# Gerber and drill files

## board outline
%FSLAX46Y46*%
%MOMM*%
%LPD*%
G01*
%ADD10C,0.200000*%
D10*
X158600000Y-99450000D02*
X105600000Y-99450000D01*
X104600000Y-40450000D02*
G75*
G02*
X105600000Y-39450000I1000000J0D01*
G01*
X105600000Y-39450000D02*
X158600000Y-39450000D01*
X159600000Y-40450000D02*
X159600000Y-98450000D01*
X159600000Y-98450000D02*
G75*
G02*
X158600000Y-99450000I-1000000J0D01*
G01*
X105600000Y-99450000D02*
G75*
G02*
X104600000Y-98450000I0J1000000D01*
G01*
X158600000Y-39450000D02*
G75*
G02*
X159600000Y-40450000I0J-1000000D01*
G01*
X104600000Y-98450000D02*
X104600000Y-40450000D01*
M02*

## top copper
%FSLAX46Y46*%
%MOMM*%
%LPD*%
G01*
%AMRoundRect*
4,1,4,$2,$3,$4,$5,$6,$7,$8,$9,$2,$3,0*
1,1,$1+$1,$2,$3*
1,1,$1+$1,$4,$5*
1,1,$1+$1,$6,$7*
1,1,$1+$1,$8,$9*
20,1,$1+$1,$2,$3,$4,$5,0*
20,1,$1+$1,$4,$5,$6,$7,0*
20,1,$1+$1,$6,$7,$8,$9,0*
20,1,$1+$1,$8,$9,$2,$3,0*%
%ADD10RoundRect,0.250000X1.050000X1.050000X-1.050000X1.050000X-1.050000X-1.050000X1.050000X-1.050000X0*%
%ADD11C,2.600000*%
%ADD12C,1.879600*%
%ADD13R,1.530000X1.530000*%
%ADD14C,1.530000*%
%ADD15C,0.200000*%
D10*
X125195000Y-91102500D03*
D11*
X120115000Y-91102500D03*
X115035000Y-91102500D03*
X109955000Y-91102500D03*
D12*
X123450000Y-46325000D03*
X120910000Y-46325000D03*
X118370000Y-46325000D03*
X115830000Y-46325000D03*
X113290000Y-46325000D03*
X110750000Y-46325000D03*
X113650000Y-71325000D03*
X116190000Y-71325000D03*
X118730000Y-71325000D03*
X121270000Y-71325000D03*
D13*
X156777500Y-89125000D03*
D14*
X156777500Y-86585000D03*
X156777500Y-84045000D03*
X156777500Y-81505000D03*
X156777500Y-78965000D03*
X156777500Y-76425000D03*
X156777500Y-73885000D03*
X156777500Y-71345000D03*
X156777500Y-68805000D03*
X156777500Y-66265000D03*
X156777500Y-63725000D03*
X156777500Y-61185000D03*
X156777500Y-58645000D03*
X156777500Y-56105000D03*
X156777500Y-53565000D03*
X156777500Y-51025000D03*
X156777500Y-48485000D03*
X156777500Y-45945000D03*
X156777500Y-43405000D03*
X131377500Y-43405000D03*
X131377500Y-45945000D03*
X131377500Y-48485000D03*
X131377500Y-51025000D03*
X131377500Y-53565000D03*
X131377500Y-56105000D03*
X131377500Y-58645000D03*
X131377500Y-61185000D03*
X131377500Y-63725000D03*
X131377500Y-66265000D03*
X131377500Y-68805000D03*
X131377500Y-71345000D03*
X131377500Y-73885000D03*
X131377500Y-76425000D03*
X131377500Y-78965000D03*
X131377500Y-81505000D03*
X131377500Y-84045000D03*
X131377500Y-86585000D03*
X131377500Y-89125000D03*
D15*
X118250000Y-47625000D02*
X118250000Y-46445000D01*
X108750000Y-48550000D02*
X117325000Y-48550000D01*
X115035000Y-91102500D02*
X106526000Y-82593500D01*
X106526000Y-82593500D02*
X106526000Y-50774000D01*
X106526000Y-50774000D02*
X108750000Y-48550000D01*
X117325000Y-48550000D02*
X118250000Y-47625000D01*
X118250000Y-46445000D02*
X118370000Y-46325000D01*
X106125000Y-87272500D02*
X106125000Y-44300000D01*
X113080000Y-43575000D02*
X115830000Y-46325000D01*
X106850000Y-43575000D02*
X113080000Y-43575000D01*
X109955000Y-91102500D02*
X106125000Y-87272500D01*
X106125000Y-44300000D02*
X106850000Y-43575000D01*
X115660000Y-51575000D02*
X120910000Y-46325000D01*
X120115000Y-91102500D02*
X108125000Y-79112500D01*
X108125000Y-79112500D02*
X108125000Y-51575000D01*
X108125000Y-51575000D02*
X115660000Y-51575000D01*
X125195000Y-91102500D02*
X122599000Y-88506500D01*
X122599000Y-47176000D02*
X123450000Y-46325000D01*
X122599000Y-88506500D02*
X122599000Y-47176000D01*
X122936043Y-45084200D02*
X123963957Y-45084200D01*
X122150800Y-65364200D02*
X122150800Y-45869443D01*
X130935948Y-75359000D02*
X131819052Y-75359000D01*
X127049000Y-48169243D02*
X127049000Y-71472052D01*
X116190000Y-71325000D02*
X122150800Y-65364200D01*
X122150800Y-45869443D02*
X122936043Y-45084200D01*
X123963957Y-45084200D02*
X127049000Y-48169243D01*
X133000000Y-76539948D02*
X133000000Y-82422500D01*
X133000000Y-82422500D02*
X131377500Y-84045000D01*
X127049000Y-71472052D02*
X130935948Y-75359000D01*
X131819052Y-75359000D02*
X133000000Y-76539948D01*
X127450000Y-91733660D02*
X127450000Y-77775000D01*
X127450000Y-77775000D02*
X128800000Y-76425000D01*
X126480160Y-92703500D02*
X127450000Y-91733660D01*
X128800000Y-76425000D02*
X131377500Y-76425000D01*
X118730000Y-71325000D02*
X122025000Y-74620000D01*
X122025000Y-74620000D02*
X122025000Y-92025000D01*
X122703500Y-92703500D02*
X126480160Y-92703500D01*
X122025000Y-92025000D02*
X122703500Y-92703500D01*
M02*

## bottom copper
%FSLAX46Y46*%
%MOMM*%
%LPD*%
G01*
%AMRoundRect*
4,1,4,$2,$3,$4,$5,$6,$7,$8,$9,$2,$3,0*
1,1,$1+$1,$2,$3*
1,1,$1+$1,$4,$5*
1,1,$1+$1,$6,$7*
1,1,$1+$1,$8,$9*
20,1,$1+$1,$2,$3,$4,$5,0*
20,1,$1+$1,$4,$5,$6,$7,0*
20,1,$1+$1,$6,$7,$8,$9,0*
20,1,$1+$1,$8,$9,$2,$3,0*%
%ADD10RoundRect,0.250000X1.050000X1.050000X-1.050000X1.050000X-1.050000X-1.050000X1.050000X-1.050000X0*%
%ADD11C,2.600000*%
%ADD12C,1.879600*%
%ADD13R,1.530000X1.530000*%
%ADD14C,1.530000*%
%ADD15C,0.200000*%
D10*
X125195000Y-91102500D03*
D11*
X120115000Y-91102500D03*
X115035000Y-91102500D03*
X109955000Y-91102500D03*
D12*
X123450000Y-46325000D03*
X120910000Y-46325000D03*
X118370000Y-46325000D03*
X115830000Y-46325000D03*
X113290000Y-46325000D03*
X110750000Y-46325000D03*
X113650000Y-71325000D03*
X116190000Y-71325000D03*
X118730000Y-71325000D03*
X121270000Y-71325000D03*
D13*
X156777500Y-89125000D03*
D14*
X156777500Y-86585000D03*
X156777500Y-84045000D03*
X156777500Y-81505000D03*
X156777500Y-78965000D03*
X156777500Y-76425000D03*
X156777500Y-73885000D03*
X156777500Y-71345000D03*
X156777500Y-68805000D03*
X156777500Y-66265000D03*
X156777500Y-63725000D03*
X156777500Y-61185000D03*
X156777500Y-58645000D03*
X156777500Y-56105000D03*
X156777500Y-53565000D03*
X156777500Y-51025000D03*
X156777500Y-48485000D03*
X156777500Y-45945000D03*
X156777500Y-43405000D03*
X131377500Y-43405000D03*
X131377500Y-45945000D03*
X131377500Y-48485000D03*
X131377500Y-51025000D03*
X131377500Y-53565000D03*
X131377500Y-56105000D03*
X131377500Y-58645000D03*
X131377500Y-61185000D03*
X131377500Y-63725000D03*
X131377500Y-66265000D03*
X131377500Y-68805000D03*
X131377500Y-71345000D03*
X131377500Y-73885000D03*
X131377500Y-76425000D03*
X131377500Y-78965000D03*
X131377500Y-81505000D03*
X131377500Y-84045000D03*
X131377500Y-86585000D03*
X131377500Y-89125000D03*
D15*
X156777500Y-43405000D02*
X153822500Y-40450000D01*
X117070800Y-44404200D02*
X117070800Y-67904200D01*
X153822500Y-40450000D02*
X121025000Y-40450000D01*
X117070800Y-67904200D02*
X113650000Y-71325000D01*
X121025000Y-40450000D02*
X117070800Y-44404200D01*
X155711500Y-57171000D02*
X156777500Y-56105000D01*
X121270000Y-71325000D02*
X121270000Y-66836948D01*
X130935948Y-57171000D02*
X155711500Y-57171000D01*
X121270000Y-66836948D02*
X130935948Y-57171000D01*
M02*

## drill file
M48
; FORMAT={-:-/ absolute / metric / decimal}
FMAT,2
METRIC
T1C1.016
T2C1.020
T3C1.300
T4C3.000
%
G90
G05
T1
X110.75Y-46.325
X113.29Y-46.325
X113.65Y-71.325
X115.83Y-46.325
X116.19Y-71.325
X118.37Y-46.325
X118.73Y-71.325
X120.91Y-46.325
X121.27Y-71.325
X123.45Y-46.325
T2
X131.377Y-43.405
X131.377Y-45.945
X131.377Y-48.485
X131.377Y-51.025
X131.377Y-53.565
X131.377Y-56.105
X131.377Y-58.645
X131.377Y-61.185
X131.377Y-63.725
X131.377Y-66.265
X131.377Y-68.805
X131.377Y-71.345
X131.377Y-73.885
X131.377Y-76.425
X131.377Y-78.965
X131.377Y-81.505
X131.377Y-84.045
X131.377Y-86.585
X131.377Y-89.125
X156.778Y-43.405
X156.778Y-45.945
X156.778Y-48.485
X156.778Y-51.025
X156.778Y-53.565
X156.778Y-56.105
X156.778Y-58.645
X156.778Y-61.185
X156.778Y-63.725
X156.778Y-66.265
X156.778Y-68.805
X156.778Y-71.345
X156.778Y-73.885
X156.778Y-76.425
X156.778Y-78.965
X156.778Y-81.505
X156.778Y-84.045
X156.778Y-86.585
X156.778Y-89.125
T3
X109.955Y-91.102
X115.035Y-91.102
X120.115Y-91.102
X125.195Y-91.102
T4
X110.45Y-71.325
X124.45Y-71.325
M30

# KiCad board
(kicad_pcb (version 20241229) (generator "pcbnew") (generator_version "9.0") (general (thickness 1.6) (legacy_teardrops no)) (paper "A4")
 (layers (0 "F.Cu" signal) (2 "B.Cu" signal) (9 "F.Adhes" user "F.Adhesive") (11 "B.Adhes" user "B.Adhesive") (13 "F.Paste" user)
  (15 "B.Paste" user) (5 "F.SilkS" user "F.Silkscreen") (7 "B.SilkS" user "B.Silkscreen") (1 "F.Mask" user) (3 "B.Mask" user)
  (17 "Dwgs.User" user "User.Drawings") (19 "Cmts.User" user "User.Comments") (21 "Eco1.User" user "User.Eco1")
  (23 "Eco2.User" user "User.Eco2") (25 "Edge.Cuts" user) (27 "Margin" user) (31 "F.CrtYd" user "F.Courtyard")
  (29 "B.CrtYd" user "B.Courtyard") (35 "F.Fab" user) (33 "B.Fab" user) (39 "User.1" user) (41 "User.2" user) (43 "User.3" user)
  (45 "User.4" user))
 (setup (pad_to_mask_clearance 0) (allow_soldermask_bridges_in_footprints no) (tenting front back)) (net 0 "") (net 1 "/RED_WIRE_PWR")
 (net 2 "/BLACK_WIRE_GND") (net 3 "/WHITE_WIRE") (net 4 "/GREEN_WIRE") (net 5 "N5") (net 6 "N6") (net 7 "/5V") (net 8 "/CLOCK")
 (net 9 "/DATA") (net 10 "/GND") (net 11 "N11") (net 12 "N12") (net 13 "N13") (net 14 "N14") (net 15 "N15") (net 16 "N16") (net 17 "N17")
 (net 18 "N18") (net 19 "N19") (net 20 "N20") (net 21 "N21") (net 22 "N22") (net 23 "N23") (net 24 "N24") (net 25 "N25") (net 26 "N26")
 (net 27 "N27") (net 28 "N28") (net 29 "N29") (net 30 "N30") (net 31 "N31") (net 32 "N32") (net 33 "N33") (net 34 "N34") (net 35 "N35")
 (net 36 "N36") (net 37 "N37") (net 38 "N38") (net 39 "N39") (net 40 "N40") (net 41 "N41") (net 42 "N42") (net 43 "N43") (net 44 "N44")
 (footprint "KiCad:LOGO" (layer "F.Cu") (at 138.975 67.075)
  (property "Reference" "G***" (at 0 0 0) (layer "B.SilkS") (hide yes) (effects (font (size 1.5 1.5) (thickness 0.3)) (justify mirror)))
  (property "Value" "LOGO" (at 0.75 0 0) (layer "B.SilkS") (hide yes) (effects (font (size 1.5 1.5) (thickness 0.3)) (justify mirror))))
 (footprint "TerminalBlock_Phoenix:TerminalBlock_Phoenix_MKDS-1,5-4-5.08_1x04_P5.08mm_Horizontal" (layer "F.Cu") (at 125.195 91.1025 180)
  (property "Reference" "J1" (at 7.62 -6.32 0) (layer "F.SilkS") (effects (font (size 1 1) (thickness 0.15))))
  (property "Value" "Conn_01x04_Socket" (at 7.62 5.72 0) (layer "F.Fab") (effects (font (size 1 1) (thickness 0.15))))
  (pad "1" thru_hole roundrect (at 0 0 180) (size 2.6 2.6) (drill 1.3) (layers "*.Cu" "*.Mask") (remove_unused_layers no)
   (roundrect_rratio 0.096154) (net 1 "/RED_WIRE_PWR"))
  (pad "2" thru_hole circle (at 5.08 0 180) (size 2.6 2.6) (drill 1.3) (layers "*.Cu" "*.Mask") (remove_unused_layers no)
   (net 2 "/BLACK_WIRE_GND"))
  (pad "3" thru_hole circle (at 10.16 0 180) (size 2.6 2.6) (drill 1.3) (layers "*.Cu" "*.Mask") (remove_unused_layers no)
   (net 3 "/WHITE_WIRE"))
  (pad "4" thru_hole circle (at 15.24 0 180) (size 2.6 2.6) (drill 1.3) (layers "*.Cu" "*.Mask") (remove_unused_layers no)
   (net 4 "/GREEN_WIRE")))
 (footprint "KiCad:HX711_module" (layer "F.Cu") (at 117.45 59.325 -90)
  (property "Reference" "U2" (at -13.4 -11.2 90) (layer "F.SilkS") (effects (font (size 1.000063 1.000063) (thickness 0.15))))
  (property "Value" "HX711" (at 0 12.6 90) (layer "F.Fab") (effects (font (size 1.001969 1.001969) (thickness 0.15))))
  (pad "" np_thru_hole circle (at 12 -7 270) (size 3 3) (drill 3) (layers "*.Cu" "*.Mask"))
  (pad "" np_thru_hole circle (at 12 7 270) (size 3 3) (drill 3) (layers "*.Cu" "*.Mask"))
  (pad "1" thru_hole circle (at -13 -6 270) (size 1.8796 1.8796) (drill 1.016) (layers "*.Cu" "*.Mask") (remove_unused_layers no)
   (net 1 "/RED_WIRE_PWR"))
  (pad "2" thru_hole circle (at -13 -3.46 270) (size 1.8796 1.8796) (drill 1.016) (layers "*.Cu" "*.Mask") (remove_unused_layers no)
   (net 2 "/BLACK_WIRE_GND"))
  (pad "3" thru_hole circle (at -13 -0.92 270) (size 1.8796 1.8796) (drill 1.016) (layers "*.Cu" "*.Mask") (remove_unused_layers no)
   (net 3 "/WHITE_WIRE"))
  (pad "4" thru_hole circle (at -13 1.62 270) (size 1.8796 1.8796) (drill 1.016) (layers "*.Cu" "*.Mask") (remove_unused_layers no)
   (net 4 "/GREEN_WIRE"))
  (pad "5" thru_hole circle (at -13 4.16 270) (size 1.8796 1.8796) (drill 1.016) (layers "*.Cu" "*.Mask") (remove_unused_layers no)
   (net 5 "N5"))
  (pad "6" thru_hole circle (at -13 6.7 270) (size 1.8796 1.8796) (drill 1.016) (layers "*.Cu" "*.Mask") (remove_unused_layers no)
   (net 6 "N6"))
  (pad "7" thru_hole circle (at 12 3.8 270) (size 1.8796 1.8796) (drill 1.016) (layers "*.Cu" "*.Mask") (remove_unused_layers no)
   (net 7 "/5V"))
  (pad "8" thru_hole circle (at 12 1.26 270) (size 1.8796 1.8796) (drill 1.016) (layers "*.Cu" "*.Mask") (remove_unused_layers no)
   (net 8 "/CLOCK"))
  (pad "9" thru_hole circle (at 12 -1.28 270) (size 1.8796 1.8796) (drill 1.016) (layers "*.Cu" "*.Mask") (remove_unused_layers no)
   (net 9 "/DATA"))
  (pad "10" thru_hole circle (at 12 -3.82 270) (size 1.8796 1.8796) (drill 1.016) (layers "*.Cu" "*.Mask") (remove_unused_layers no)
   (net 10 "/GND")))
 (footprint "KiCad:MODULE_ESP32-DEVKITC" (layer "F.Cu") (at 144.0775 66.275 180)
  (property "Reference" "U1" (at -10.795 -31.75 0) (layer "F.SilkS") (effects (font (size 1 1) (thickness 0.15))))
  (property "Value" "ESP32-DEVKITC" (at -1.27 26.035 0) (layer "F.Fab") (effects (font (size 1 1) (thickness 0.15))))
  (pad "1" thru_hole rect (at -12.7 -22.85 180) (size 1.53 1.53) (drill 1.02) (layers "*.Cu" "*.Mask") (remove_unused_layers no)
   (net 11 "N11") (solder_mask_margin 0.102))
  (pad "2" thru_hole circle (at -12.7 -20.31 180) (size 1.53 1.53) (drill 1.02) (layers "*.Cu" "*.Mask") (remove_unused_layers no)
   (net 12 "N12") (solder_mask_margin 0.102))
  (pad "3" thru_hole circle (at -12.7 -17.77 180) (size 1.53 1.53) (drill 1.02) (layers "*.Cu" "*.Mask") (remove_unused_layers no)
   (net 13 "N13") (solder_mask_margin 0.102))
  (pad "4" thru_hole circle (at -12.7 -15.23 180) (size 1.53 1.53) (drill 1.02) (layers "*.Cu" "*.Mask") (remove_unused_layers no)
   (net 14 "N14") (solder_mask_margin 0.102))
  (pad "5" thru_hole circle (at -12.7 -12.69 180) (size 1.53 1.53) (drill 1.02) (layers "*.Cu" "*.Mask") (remove_unused_layers no)
   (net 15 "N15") (solder_mask_margin 0.102))
  (pad "6" thru_hole circle (at -12.7 -10.15 180) (size 1.53 1.53) (drill 1.02) (layers "*.Cu" "*.Mask") (remove_unused_layers no)
   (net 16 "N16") (solder_mask_margin 0.102))
  (pad "7" thru_hole circle (at -12.7 -7.61 180) (size 1.53 1.53) (drill 1.02) (layers "*.Cu" "*.Mask") (remove_unused_layers no)
   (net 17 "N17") (solder_mask_margin 0.102))
  (pad "8" thru_hole circle (at -12.7 -5.07 180) (size 1.53 1.53) (drill 1.02) (layers "*.Cu" "*.Mask") (remove_unused_layers no)
   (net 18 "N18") (solder_mask_margin 0.102))
  (pad "9" thru_hole circle (at -12.7 -2.53 180) (size 1.53 1.53) (drill 1.02) (layers "*.Cu" "*.Mask") (remove_unused_layers no)
   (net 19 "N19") (solder_mask_margin 0.102))
  (pad "10" thru_hole circle (at -12.7 0.01 180) (size 1.53 1.53) (drill 1.02) (layers "*.Cu" "*.Mask") (remove_unused_layers no)
   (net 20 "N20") (solder_mask_margin 0.102))
  (pad "11" thru_hole circle (at -12.7 2.55 180) (size 1.53 1.53) (drill 1.02) (layers "*.Cu" "*.Mask") (remove_unused_layers no)
   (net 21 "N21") (solder_mask_margin 0.102))
  (pad "12" thru_hole circle (at -12.7 5.09 180) (size 1.53 1.53) (drill 1.02) (layers "*.Cu" "*.Mask") (remove_unused_layers no)
   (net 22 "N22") (solder_mask_margin 0.102))
  (pad "13" thru_hole circle (at -12.7 7.63 180) (size 1.53 1.53) (drill 1.02) (layers "*.Cu" "*.Mask") (remove_unused_layers no)
   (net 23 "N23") (solder_mask_margin 0.102))
  (pad "14" thru_hole circle (at -12.7 10.17 180) (size 1.53 1.53) (drill 1.02) (layers "*.Cu" "*.Mask") (remove_unused_layers no)
   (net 10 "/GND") (solder_mask_margin 0.102))
  (pad "15" thru_hole circle (at -12.7 12.71 180) (size 1.53 1.53) (drill 1.02) (layers "*.Cu" "*.Mask") (remove_unused_layers no)
   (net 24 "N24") (solder_mask_margin 0.102))
  (pad "16" thru_hole circle (at -12.7 15.25 180) (size 1.53 1.53) (drill 1.02) (layers "*.Cu" "*.Mask") (remove_unused_layers no)
   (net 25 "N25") (solder_mask_margin 0.102))
  (pad "17" thru_hole circle (at -12.7 17.79 180) (size 1.53 1.53) (drill 1.02) (layers "*.Cu" "*.Mask") (remove_unused_layers no)
   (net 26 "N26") (solder_mask_margin 0.102))
  (pad "18" thru_hole circle (at -12.7 20.33 180) (size 1.53 1.53) (drill 1.02) (layers "*.Cu" "*.Mask") (remove_unused_layers no)
   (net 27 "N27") (solder_mask_margin 0.102))
  (pad "19" thru_hole circle (at -12.7 22.87 180) (size 1.53 1.53) (drill 1.02) (layers "*.Cu" "*.Mask") (remove_unused_layers no)
   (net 7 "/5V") (solder_mask_margin 0.102))
  (pad "20" thru_hole circle (at 12.7 22.87 180) (size 1.53 1.53) (drill 1.02) (layers "*.Cu" "*.Mask") (remove_unused_layers no)
   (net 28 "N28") (solder_mask_margin 0.102))
  (pad "21" thru_hole circle (at 12.7 20.33 180) (size 1.53 1.53) (drill 1.02) (layers "*.Cu" "*.Mask") (remove_unused_layers no)
   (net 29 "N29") (solder_mask_margin 0.102))
  (pad "22" thru_hole circle (at 12.7 17.79 180) (size 1.53 1.53) (drill 1.02) (layers "*.Cu" "*.Mask") (remove_unused_layers no)
   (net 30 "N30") (solder_mask_margin 0.102))
  (pad "23" thru_hole circle (at 12.7 15.25 180) (size 1.53 1.53) (drill 1.02) (layers "*.Cu" "*.Mask") (remove_unused_layers no)
   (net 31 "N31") (solder_mask_margin 0.102))
  (pad "24" thru_hole circle (at 12.7 12.71 180) (size 1.53 1.53) (drill 1.02) (layers "*.Cu" "*.Mask") (remove_unused_layers no)
   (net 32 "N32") (solder_mask_margin 0.102))
  (pad "25" thru_hole circle (at 12.7 10.17 180) (size 1.53 1.53) (drill 1.02) (layers "*.Cu" "*.Mask") (remove_unused_layers no)
   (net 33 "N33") (solder_mask_margin 0.102))
  (pad "26" thru_hole circle (at 12.7 7.63 180) (size 1.53 1.53) (drill 1.02) (layers "*.Cu" "*.Mask") (remove_unused_layers no)
   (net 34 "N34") (solder_mask_margin 0.102))
  (pad "27" thru_hole circle (at 12.7 5.09 180) (size 1.53 1.53) (drill 1.02) (layers "*.Cu" "*.Mask") (remove_unused_layers no)
   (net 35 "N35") (solder_mask_margin 0.102))
  (pad "28" thru_hole circle (at 12.7 2.55 180) (size 1.53 1.53) (drill 1.02) (layers "*.Cu" "*.Mask") (remove_unused_layers no)
   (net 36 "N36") (solder_mask_margin 0.102))
  (pad "29" thru_hole circle (at 12.7 0.01 180) (size 1.53 1.53) (drill 1.02) (layers "*.Cu" "*.Mask") (remove_unused_layers no)
   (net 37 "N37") (solder_mask_margin 0.102))
  (pad "30" thru_hole circle (at 12.7 -2.53 180) (size 1.53 1.53) (drill 1.02) (layers "*.Cu" "*.Mask") (remove_unused_layers no)
   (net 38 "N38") (solder_mask_margin 0.102))
  (pad "31" thru_hole circle (at 12.7 -5.07 180) (size 1.53 1.53) (drill 1.02) (layers "*.Cu" "*.Mask") (remove_unused_layers no)
   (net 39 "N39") (solder_mask_margin 0.102))
  (pad "32" thru_hole circle (at 12.7 -7.61 180) (size 1.53 1.53) (drill 1.02) (layers "*.Cu" "*.Mask") (remove_unused_layers no)
   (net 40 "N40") (solder_mask_margin 0.102))
  (pad "33" thru_hole circle (at 12.7 -10.15 180) (size 1.53 1.53) (drill 1.02) (layers "*.Cu" "*.Mask") (remove_unused_layers no)
   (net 9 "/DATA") (solder_mask_margin 0.102))
  (pad "34" thru_hole circle (at 12.7 -12.69 180) (size 1.53 1.53) (drill 1.02) (layers "*.Cu" "*.Mask") (remove_unused_layers no)
   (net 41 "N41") (solder_mask_margin 0.102))
  (pad "35" thru_hole circle (at 12.7 -15.23 180) (size 1.53 1.53) (drill 1.02) (layers "*.Cu" "*.Mask") (remove_unused_layers no)
   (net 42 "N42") (solder_mask_margin 0.102))
  (pad "36" thru_hole circle (at 12.7 -17.77 180) (size 1.53 1.53) (drill 1.02) (layers "*.Cu" "*.Mask") (remove_unused_layers no)
   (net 8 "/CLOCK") (solder_mask_margin 0.102))
  (pad "37" thru_hole circle (at 12.7 -20.31 180) (size 1.53 1.53) (drill 1.02) (layers "*.Cu" "*.Mask") (remove_unused_layers no)
   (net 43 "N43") (solder_mask_margin 0.102))
  (pad "38" thru_hole circle (at 12.7 -22.85 180) (size 1.53 1.53) (drill 1.02) (layers "*.Cu" "*.Mask") (remove_unused_layers no)
   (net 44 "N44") (solder_mask_margin 0.102)))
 (gr_line (start 158.6 99.45) (end 105.6 99.45) (stroke (width 0.2) (type default)) (layer "Edge.Cuts"))
 (gr_arc (start 104.6 40.45) (mid 104.892893 39.742893) (end 105.6 39.45) (stroke (width 0.2) (type default)) (layer "Edge.Cuts"))
 (gr_line (start 105.6 39.45) (end 158.6 39.45) (stroke (width 0.2) (type default)) (layer "Edge.Cuts"))
 (gr_line (start 159.6 40.45) (end 159.6 98.45) (stroke (width 0.2) (type default)) (layer "Edge.Cuts"))
 (gr_arc (start 159.6 98.45) (mid 159.307107 99.157107) (end 158.6 99.45) (stroke (width 0.2) (type default)) (layer "Edge.Cuts"))
 (gr_arc (start 105.6 99.45) (mid 104.892893 99.157107) (end 104.6 98.45) (stroke (width 0.2) (type default)) (layer "Edge.Cuts"))
 (gr_arc (start 158.6 39.45) (mid 159.307107 39.742893) (end 159.6 40.45) (stroke (width 0.2) (type default)) (layer "Edge.Cuts"))
 (gr_line (start 104.6 98.45) (end 104.6 40.45) (stroke (width 0.2) (type default)) (layer "Edge.Cuts"))
 (segment (start 118.25 47.625) (end 118.25 46.445) (width 0.2) (layer "F.Cu") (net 3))
 (segment (start 108.75 48.55) (end 117.325 48.55) (width 0.2) (layer "F.Cu") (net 3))
 (segment (start 115.035 91.1025) (end 106.526 82.5935) (width 0.2) (layer "F.Cu") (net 3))
 (segment (start 106.526 82.5935) (end 106.526 50.774) (width 0.2) (layer "F.Cu") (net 3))
 (segment (start 106.526 50.774) (end 108.75 48.55) (width 0.2) (layer "F.Cu") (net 3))
 (segment (start 117.325 48.55) (end 118.25 47.625) (width 0.2) (layer "F.Cu") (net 3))
 (segment (start 118.25 46.445) (end 118.37 46.325) (width 0.2) (layer "F.Cu") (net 3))
 (segment (start 106.125 87.2725) (end 106.125 44.3) (width 0.2) (layer "F.Cu") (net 4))
 (segment (start 113.08 43.575) (end 115.83 46.325) (width 0.2) (layer "F.Cu") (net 4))
 (segment (start 106.85 43.575) (end 113.08 43.575) (width 0.2) (layer "F.Cu") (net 4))
 (segment (start 109.955 91.1025) (end 106.125 87.2725) (width 0.2) (layer "F.Cu") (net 4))
 (segment (start 106.125 44.3) (end 106.85 43.575) (width 0.2) (layer "F.Cu") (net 4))
 (segment (start 115.66 51.575) (end 120.91 46.325) (width 0.2) (layer "F.Cu") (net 2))
 (segment (start 120.115 91.1025) (end 108.125 79.1125) (width 0.2) (layer "F.Cu") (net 2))
 (segment (start 108.125 79.1125) (end 108.125 51.575) (width 0.2) (layer "F.Cu") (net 2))
 (segment (start 108.125 51.575) (end 115.66 51.575) (width 0.2) (layer "F.Cu") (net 2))
 (segment (start 125.195 91.1025) (end 122.599 88.5065) (width 0.2) (layer "F.Cu") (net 1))
 (segment (start 122.599 47.176) (end 123.45 46.325) (width 0.2) (layer "F.Cu") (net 1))
 (segment (start 122.599 88.5065) (end 122.599 47.176) (width 0.2) (layer "F.Cu") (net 1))
 (segment (start 156.7775 43.405) (end 153.8225 40.45) (width 0.2) (layer "B.Cu") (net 7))
 (segment (start 117.0708 44.4042) (end 117.0708 67.9042) (width 0.2) (layer "B.Cu") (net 7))
 (segment (start 153.8225 40.45) (end 121.025 40.45) (width 0.2) (layer "B.Cu") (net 7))
 (segment (start 117.0708 67.9042) (end 113.65 71.325) (width 0.2) (layer "B.Cu") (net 7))
 (segment (start 121.025 40.45) (end 117.0708 44.4042) (width 0.2) (layer "B.Cu") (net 7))
 (segment (start 122.936043 45.0842) (end 123.963957 45.0842) (width 0.2) (layer "F.Cu") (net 8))
 (segment (start 122.1508 65.3642) (end 122.1508 45.869443) (width 0.2) (layer "F.Cu") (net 8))
 (segment (start 130.935948 75.359) (end 131.819052 75.359) (width 0.2) (layer "F.Cu") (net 8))
 (segment (start 127.049 48.169243) (end 127.049 71.472052) (width 0.2) (layer "F.Cu") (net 8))
 (segment (start 116.19 71.325) (end 122.1508 65.3642) (width 0.2) (layer "F.Cu") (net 8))
 (segment (start 122.1508 45.869443) (end 122.936043 45.0842) (width 0.2) (layer "F.Cu") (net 8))
 (segment (start 123.963957 45.0842) (end 127.049 48.169243) (width 0.2) (layer "F.Cu") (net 8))
 (segment (start 133 76.539948) (end 133 82.4225) (width 0.2) (layer "F.Cu") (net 8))
 (segment (start 133 82.4225) (end 131.3775 84.045) (width 0.2) (layer "F.Cu") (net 8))
 (segment (start 127.049 71.472052) (end 130.935948 75.359) (width 0.2) (layer "F.Cu") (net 8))
 (segment (start 131.819052 75.359) (end 133 76.539948) (width 0.2) (layer "F.Cu") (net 8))
 (segment (start 127.45 91.73366) (end 127.45 77.775) (width 0.2) (layer "F.Cu") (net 9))
 (segment (start 127.45 77.775) (end 128.8 76.425) (width 0.2) (layer "F.Cu") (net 9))
 (segment (start 126.48016 92.7035) (end 127.45 91.73366) (width 0.2) (layer "F.Cu") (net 9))
 (segment (start 128.8 76.425) (end 131.3775 76.425) (width 0.2) (layer "F.Cu") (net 9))
 (segment (start 118.73 71.325) (end 122.025 74.62) (width 0.2) (layer "F.Cu") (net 9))
 (segment (start 122.025 74.62) (end 122.025 92.025) (width 0.2) (layer "F.Cu") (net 9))
 (segment (start 122.7035 92.7035) (end 126.48016 92.7035) (width 0.2) (layer "F.Cu") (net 9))
 (segment (start 122.025 92.025) (end 122.7035 92.7035) (width 0.2) (layer "F.Cu") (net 9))
 (segment (start 155.7115 57.171) (end 156.7775 56.105) (width 0.2) (layer "B.Cu") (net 10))
 (segment (start 121.27 71.325) (end 121.27 66.836948) (width 0.2) (layer "B.Cu") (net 10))
 (segment (start 130.935948 57.171) (end 155.7115 57.171) (width 0.2) (layer "B.Cu") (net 10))
 (segment (start 121.27 66.836948) (end 130.935948 57.171) (width 0.2) (layer "B.Cu") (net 10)))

